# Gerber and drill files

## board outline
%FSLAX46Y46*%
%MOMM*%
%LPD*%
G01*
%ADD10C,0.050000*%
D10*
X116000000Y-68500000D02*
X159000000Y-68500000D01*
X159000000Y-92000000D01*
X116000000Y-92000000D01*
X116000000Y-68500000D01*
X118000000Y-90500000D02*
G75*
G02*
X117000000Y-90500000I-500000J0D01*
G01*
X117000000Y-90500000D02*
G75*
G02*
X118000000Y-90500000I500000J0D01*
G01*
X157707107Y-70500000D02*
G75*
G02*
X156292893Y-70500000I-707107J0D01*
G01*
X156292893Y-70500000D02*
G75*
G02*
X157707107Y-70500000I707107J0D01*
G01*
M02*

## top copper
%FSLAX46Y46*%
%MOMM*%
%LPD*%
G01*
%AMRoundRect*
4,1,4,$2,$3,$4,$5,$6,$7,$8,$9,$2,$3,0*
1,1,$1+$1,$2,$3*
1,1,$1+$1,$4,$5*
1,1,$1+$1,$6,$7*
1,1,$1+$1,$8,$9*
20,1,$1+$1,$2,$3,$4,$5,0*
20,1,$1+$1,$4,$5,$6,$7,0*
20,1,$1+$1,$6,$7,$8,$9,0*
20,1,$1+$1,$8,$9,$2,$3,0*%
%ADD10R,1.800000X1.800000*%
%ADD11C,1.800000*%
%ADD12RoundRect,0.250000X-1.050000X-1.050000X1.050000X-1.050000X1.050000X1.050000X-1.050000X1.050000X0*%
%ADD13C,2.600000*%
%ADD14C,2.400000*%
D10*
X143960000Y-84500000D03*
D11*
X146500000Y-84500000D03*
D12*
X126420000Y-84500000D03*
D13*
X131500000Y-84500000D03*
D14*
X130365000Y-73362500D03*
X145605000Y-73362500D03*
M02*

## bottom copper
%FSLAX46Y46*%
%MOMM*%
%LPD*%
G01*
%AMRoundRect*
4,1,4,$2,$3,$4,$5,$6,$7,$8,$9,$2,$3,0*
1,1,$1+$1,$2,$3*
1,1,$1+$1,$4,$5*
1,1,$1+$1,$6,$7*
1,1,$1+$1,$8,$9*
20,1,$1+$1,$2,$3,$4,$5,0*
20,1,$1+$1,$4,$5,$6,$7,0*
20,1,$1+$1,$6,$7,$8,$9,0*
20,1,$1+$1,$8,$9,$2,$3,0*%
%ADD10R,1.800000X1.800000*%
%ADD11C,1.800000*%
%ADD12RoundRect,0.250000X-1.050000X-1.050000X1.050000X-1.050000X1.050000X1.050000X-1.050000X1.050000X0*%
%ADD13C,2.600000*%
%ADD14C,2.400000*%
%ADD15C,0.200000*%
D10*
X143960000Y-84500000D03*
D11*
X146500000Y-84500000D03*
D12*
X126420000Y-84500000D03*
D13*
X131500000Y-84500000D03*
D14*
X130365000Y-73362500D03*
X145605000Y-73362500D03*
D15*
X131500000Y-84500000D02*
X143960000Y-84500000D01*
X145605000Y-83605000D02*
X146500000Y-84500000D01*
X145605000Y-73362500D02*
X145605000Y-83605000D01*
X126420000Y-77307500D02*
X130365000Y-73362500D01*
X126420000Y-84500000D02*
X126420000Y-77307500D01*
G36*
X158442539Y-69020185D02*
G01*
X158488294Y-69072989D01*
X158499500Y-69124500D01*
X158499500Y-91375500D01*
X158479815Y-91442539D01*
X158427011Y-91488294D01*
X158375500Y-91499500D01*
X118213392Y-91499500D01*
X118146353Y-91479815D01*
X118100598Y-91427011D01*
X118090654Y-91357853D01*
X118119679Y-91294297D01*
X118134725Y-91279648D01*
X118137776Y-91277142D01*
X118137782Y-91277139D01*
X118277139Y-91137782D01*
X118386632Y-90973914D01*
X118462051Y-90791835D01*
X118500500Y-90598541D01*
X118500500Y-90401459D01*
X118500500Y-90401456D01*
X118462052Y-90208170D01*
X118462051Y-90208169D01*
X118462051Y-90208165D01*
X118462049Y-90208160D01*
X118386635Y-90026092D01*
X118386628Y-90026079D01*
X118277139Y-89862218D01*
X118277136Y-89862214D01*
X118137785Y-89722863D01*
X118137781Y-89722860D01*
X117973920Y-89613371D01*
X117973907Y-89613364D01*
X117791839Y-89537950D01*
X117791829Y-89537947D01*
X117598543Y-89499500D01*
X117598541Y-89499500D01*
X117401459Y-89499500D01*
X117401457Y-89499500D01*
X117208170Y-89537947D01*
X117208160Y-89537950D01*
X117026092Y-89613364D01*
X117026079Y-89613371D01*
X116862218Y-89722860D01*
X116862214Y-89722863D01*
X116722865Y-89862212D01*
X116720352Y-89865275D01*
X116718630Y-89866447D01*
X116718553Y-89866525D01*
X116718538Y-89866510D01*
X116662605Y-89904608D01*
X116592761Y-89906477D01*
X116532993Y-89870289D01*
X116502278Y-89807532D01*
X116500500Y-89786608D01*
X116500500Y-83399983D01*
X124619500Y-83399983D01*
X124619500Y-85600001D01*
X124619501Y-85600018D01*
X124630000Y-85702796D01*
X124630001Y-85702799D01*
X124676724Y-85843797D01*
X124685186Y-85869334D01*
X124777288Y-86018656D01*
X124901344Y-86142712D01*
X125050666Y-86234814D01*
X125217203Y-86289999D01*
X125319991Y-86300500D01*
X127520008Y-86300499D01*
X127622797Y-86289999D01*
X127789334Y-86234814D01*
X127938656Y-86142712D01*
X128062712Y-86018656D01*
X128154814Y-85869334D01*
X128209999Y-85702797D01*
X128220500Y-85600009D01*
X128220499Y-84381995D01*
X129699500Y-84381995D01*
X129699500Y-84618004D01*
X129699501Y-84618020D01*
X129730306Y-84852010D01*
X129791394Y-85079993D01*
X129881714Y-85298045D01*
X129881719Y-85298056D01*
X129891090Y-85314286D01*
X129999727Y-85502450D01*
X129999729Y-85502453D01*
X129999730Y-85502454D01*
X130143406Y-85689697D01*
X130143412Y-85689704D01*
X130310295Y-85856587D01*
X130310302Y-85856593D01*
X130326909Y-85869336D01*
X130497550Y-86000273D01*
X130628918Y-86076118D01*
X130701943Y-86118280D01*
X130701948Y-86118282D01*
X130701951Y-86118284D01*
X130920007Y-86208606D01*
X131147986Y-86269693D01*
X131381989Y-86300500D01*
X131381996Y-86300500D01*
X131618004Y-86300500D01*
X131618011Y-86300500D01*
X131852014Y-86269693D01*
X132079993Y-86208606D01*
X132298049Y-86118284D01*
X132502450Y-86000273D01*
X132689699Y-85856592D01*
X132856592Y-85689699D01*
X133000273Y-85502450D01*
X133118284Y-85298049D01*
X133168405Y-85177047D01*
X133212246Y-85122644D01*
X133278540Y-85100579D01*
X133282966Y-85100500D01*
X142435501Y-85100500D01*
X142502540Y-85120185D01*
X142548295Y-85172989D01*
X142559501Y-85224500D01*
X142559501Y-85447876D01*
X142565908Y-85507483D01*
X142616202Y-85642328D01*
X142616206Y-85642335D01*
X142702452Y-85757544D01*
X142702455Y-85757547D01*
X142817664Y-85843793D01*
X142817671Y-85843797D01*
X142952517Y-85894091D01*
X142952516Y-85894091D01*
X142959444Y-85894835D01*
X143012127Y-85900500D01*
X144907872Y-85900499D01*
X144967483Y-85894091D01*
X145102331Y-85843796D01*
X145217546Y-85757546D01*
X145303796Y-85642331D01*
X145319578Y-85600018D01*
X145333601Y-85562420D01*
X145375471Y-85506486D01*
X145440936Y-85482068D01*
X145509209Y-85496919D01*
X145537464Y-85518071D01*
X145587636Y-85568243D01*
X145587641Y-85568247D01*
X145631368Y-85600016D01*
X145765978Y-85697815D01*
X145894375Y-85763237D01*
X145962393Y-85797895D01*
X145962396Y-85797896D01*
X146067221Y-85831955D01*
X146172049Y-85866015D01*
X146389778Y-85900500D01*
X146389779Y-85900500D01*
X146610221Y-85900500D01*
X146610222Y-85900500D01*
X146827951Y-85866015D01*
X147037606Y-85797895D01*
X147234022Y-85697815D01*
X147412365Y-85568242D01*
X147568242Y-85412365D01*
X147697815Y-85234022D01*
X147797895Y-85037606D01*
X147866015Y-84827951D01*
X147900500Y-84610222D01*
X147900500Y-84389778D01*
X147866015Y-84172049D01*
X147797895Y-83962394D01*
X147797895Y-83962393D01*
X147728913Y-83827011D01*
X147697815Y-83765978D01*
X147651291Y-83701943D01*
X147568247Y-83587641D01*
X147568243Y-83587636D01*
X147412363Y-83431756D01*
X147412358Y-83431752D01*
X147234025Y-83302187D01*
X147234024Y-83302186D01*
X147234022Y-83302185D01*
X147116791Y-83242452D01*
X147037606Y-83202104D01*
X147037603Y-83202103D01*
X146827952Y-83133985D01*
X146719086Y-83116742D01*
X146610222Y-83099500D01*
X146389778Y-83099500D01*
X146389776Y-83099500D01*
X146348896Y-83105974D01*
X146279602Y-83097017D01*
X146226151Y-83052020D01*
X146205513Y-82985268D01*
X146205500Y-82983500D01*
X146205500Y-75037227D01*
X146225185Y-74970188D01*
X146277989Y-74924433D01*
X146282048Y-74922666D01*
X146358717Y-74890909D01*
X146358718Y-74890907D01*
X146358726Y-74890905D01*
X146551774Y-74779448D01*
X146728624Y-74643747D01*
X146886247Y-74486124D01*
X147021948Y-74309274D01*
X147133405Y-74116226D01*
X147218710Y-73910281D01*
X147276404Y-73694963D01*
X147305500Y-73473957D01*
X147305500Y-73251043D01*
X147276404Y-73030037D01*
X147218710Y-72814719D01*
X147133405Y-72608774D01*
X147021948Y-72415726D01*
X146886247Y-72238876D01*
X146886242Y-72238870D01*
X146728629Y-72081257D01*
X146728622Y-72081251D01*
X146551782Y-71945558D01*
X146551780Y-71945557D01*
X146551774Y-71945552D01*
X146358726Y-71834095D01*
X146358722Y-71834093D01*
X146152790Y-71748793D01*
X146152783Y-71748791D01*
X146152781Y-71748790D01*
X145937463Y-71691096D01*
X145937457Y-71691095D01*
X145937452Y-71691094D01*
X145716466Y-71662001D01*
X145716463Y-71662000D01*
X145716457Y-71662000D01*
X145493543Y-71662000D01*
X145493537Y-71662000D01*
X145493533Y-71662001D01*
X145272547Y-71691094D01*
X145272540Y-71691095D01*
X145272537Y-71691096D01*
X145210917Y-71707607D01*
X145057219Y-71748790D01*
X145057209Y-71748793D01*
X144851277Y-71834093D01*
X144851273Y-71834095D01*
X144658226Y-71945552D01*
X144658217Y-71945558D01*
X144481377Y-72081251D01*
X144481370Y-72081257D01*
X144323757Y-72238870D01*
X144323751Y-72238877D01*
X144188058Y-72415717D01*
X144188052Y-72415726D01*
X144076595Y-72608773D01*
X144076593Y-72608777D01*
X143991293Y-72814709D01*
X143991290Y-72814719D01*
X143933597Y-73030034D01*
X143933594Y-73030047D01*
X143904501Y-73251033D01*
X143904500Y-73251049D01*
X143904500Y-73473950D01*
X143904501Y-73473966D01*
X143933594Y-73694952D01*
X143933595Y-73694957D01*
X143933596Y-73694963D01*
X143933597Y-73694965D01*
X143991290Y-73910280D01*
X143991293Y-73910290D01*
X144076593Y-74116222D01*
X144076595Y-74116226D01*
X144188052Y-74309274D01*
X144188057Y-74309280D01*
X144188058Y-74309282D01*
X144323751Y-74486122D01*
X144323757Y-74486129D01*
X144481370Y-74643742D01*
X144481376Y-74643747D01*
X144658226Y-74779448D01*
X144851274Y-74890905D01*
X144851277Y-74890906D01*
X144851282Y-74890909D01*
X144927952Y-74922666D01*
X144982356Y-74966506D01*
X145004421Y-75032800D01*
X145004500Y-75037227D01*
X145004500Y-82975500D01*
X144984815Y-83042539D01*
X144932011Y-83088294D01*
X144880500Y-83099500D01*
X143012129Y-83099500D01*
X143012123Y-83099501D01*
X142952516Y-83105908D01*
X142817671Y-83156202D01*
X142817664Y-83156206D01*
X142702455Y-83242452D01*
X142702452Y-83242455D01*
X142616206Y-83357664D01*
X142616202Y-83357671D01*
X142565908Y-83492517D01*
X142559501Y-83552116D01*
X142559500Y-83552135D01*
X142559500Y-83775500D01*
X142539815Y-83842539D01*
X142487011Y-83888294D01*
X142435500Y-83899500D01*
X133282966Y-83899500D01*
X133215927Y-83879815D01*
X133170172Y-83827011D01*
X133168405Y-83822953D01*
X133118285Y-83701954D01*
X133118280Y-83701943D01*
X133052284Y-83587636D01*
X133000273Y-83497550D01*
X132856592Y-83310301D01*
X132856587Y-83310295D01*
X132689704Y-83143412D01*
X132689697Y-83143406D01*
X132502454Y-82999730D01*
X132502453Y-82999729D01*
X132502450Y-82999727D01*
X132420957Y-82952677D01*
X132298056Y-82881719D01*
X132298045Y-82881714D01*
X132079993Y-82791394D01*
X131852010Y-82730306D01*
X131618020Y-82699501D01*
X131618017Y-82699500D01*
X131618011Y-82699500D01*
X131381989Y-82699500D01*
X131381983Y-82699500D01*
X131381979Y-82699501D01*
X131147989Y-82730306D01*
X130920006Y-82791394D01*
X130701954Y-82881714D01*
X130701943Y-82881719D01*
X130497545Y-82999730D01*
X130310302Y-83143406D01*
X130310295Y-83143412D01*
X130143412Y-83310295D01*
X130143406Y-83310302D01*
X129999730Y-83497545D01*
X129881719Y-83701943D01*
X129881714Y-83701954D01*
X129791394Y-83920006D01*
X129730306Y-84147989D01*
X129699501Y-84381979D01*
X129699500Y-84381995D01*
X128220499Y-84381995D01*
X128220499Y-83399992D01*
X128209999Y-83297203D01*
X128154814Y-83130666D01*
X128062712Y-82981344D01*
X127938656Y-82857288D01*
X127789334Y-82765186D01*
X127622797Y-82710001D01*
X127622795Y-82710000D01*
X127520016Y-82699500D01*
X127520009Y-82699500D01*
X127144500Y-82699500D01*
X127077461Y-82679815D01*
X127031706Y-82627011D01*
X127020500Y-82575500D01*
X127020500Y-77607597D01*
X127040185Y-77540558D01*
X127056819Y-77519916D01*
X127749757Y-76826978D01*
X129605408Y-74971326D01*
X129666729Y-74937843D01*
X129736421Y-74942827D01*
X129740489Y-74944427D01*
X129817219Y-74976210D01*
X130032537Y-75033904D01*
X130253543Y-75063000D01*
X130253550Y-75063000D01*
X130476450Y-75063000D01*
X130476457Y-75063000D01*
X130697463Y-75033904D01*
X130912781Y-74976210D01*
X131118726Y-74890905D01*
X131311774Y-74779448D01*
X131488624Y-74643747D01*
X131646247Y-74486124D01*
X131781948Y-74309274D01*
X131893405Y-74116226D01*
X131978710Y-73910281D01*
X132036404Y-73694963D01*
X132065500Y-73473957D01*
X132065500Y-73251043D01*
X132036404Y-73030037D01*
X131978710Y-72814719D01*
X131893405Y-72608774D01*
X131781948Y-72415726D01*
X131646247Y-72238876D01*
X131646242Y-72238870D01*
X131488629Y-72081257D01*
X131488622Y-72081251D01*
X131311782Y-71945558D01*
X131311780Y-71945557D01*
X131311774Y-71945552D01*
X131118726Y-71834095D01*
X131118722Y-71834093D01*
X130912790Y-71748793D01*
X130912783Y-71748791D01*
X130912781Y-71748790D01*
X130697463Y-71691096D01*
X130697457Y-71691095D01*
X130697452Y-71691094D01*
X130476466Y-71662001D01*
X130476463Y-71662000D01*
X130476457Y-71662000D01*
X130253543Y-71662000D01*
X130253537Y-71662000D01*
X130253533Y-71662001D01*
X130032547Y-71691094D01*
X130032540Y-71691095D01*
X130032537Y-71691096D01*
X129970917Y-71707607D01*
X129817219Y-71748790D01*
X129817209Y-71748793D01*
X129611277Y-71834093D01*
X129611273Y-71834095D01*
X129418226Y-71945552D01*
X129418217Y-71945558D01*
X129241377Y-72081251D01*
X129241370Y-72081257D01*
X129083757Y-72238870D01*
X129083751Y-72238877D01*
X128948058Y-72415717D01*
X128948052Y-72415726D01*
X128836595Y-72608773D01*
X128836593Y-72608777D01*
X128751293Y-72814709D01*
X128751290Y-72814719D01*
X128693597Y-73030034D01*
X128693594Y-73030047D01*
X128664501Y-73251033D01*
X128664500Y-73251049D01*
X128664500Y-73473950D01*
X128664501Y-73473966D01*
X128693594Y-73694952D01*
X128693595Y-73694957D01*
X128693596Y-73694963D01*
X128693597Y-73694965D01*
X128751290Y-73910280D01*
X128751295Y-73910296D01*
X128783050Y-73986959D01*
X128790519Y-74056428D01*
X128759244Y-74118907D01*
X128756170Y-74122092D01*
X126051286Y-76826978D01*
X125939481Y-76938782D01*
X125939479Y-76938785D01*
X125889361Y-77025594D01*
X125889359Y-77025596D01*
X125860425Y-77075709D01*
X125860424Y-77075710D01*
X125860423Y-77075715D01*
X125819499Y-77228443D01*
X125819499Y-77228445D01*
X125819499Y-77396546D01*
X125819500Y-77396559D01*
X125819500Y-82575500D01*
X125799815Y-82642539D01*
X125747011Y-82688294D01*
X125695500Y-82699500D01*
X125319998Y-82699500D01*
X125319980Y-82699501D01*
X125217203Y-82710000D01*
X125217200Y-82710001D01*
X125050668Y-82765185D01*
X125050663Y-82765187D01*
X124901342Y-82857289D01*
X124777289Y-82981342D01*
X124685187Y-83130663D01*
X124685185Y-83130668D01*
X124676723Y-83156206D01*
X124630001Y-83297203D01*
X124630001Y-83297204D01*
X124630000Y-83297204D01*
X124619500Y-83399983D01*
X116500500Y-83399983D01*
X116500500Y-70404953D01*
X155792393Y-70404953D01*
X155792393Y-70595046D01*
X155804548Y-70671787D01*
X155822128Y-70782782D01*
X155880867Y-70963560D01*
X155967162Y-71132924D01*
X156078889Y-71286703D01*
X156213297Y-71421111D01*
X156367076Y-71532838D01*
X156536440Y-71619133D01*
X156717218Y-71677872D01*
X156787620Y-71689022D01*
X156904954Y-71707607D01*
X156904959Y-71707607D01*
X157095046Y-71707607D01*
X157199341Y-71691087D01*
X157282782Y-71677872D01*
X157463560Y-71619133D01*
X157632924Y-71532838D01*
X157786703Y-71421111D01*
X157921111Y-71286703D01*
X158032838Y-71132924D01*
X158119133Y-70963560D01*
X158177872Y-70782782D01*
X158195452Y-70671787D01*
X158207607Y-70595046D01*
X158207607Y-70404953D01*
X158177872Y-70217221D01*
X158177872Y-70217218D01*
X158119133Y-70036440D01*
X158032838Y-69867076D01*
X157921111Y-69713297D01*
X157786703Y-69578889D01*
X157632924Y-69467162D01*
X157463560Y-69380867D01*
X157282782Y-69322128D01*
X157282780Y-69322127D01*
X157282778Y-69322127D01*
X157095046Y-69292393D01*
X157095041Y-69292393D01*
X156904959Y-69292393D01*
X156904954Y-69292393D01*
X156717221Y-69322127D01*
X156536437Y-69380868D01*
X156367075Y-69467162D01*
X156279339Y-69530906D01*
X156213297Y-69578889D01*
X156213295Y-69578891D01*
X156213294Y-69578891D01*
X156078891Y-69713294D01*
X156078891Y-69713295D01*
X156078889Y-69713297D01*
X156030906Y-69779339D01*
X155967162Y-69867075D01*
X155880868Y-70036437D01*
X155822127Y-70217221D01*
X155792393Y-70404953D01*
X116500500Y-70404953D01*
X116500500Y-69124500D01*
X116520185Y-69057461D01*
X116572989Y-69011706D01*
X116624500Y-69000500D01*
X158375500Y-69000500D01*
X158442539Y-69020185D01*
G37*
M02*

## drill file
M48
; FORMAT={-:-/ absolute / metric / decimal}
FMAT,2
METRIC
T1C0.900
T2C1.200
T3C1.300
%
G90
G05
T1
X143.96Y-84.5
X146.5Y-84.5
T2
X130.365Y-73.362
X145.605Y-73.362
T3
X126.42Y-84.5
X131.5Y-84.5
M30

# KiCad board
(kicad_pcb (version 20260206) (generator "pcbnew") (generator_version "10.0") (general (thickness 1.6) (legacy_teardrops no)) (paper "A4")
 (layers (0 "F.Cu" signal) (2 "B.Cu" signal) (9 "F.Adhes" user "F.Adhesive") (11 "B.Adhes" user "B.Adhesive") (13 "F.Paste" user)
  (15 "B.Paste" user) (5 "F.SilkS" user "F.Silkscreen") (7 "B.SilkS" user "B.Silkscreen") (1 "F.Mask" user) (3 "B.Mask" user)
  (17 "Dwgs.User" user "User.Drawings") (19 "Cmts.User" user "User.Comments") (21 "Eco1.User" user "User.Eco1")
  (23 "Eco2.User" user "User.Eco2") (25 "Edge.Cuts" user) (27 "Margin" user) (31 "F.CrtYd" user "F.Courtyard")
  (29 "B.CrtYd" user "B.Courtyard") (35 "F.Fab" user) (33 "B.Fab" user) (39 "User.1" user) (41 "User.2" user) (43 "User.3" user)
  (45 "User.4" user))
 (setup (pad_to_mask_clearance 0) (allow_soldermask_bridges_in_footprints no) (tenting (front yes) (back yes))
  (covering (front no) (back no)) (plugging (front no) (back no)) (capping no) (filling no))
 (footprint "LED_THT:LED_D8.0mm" (layer "F.Cu") (at 143.96 84.5)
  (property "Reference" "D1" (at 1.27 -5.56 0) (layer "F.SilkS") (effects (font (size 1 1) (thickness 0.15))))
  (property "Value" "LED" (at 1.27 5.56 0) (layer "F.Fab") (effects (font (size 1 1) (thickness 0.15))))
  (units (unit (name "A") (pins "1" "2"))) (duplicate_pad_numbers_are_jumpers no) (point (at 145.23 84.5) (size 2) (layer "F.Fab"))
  (pad "1" thru_hole rect (at 0 0) (size 1.8 1.8) (drill 0.9) (layers "*.Cu" "*.Mask") (remove_unused_layers no) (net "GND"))
  (pad "2" thru_hole circle (at 2.54 0) (size 1.8 1.8) (drill 0.9) (layers "*.Cu" "*.Mask") (remove_unused_layers no) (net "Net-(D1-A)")))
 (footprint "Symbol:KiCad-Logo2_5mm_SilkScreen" (layer "F.Cu") (at 137 79.5)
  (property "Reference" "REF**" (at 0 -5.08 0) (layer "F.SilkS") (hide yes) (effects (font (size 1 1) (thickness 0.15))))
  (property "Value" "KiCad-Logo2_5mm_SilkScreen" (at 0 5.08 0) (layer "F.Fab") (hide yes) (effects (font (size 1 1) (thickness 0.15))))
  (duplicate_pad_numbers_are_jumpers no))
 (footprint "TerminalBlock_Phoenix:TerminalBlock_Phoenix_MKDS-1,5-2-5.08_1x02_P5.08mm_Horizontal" (layer "F.Cu") (at 126.42 84.5)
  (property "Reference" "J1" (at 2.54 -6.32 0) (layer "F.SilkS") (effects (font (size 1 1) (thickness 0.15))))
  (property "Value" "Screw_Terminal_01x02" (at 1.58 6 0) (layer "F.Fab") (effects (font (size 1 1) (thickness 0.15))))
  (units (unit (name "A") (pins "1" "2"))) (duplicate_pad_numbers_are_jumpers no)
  (pad "1" thru_hole roundrect (at 0 0) (size 2.6 2.6) (drill 1.3) (layers "*.Cu" "*.Mask") (remove_unused_layers no)
   (roundrect_rratio 0.096154) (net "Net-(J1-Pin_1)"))
  (pad "2" thru_hole circle (at 5.08 0) (size 2.6 2.6) (drill 1.3) (layers "*.Cu" "*.Mask") (remove_unused_layers no) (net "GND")))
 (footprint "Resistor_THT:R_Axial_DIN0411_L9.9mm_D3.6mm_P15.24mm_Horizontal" (layer "F.Cu") (at 130.365 73.3625)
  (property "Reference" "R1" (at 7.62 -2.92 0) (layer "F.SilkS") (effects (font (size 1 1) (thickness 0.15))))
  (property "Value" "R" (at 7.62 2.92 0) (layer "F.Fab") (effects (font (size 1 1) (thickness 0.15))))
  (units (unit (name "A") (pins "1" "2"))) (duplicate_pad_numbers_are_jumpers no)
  (pad "1" thru_hole circle (at 0 0) (size 2.4 2.4) (drill 1.2) (layers "*.Cu" "*.Mask") (remove_unused_layers no) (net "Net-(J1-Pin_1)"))
  (pad "2" thru_hole circle (at 15.24 0) (size 2.4 2.4) (drill 1.2) (layers "*.Cu" "*.Mask") (remove_unused_layers no) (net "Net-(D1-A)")))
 (gr_rect (start 116 68.5) (end 159 92) (stroke (width 0.05) (type default)) (fill no) (layer "Edge.Cuts"))
 (gr_circle (center 117.5 90.5) (end 117.5 91) (stroke (width 0.05) (type default)) (fill no) (layer "Edge.Cuts"))
 (gr_circle (center 157 70.5) (end 157.5 71) (stroke (width 0.05) (type default)) (fill no) (layer "Edge.Cuts"))
 (segment (start 131.5 84.5) (end 143.96 84.5) (width 0.2) (layer "B.Cu") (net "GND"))
 (segment (start 145.605 83.605) (end 146.5 84.5) (width 0.2) (layer "B.Cu") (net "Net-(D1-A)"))
 (segment (start 145.605 73.3625) (end 145.605 83.605) (width 0.2) (layer "B.Cu") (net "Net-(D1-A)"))
 (segment (start 126.42 77.3075) (end 130.365 73.3625) (width 0.2) (layer "B.Cu") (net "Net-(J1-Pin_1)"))
 (segment (start 126.42 84.5) (end 126.42 77.3075) (width 0.2) (layer "B.Cu") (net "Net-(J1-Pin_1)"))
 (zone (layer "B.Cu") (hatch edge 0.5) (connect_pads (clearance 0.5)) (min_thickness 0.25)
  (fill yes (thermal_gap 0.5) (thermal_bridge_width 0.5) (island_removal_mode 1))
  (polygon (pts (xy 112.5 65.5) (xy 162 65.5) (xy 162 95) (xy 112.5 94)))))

